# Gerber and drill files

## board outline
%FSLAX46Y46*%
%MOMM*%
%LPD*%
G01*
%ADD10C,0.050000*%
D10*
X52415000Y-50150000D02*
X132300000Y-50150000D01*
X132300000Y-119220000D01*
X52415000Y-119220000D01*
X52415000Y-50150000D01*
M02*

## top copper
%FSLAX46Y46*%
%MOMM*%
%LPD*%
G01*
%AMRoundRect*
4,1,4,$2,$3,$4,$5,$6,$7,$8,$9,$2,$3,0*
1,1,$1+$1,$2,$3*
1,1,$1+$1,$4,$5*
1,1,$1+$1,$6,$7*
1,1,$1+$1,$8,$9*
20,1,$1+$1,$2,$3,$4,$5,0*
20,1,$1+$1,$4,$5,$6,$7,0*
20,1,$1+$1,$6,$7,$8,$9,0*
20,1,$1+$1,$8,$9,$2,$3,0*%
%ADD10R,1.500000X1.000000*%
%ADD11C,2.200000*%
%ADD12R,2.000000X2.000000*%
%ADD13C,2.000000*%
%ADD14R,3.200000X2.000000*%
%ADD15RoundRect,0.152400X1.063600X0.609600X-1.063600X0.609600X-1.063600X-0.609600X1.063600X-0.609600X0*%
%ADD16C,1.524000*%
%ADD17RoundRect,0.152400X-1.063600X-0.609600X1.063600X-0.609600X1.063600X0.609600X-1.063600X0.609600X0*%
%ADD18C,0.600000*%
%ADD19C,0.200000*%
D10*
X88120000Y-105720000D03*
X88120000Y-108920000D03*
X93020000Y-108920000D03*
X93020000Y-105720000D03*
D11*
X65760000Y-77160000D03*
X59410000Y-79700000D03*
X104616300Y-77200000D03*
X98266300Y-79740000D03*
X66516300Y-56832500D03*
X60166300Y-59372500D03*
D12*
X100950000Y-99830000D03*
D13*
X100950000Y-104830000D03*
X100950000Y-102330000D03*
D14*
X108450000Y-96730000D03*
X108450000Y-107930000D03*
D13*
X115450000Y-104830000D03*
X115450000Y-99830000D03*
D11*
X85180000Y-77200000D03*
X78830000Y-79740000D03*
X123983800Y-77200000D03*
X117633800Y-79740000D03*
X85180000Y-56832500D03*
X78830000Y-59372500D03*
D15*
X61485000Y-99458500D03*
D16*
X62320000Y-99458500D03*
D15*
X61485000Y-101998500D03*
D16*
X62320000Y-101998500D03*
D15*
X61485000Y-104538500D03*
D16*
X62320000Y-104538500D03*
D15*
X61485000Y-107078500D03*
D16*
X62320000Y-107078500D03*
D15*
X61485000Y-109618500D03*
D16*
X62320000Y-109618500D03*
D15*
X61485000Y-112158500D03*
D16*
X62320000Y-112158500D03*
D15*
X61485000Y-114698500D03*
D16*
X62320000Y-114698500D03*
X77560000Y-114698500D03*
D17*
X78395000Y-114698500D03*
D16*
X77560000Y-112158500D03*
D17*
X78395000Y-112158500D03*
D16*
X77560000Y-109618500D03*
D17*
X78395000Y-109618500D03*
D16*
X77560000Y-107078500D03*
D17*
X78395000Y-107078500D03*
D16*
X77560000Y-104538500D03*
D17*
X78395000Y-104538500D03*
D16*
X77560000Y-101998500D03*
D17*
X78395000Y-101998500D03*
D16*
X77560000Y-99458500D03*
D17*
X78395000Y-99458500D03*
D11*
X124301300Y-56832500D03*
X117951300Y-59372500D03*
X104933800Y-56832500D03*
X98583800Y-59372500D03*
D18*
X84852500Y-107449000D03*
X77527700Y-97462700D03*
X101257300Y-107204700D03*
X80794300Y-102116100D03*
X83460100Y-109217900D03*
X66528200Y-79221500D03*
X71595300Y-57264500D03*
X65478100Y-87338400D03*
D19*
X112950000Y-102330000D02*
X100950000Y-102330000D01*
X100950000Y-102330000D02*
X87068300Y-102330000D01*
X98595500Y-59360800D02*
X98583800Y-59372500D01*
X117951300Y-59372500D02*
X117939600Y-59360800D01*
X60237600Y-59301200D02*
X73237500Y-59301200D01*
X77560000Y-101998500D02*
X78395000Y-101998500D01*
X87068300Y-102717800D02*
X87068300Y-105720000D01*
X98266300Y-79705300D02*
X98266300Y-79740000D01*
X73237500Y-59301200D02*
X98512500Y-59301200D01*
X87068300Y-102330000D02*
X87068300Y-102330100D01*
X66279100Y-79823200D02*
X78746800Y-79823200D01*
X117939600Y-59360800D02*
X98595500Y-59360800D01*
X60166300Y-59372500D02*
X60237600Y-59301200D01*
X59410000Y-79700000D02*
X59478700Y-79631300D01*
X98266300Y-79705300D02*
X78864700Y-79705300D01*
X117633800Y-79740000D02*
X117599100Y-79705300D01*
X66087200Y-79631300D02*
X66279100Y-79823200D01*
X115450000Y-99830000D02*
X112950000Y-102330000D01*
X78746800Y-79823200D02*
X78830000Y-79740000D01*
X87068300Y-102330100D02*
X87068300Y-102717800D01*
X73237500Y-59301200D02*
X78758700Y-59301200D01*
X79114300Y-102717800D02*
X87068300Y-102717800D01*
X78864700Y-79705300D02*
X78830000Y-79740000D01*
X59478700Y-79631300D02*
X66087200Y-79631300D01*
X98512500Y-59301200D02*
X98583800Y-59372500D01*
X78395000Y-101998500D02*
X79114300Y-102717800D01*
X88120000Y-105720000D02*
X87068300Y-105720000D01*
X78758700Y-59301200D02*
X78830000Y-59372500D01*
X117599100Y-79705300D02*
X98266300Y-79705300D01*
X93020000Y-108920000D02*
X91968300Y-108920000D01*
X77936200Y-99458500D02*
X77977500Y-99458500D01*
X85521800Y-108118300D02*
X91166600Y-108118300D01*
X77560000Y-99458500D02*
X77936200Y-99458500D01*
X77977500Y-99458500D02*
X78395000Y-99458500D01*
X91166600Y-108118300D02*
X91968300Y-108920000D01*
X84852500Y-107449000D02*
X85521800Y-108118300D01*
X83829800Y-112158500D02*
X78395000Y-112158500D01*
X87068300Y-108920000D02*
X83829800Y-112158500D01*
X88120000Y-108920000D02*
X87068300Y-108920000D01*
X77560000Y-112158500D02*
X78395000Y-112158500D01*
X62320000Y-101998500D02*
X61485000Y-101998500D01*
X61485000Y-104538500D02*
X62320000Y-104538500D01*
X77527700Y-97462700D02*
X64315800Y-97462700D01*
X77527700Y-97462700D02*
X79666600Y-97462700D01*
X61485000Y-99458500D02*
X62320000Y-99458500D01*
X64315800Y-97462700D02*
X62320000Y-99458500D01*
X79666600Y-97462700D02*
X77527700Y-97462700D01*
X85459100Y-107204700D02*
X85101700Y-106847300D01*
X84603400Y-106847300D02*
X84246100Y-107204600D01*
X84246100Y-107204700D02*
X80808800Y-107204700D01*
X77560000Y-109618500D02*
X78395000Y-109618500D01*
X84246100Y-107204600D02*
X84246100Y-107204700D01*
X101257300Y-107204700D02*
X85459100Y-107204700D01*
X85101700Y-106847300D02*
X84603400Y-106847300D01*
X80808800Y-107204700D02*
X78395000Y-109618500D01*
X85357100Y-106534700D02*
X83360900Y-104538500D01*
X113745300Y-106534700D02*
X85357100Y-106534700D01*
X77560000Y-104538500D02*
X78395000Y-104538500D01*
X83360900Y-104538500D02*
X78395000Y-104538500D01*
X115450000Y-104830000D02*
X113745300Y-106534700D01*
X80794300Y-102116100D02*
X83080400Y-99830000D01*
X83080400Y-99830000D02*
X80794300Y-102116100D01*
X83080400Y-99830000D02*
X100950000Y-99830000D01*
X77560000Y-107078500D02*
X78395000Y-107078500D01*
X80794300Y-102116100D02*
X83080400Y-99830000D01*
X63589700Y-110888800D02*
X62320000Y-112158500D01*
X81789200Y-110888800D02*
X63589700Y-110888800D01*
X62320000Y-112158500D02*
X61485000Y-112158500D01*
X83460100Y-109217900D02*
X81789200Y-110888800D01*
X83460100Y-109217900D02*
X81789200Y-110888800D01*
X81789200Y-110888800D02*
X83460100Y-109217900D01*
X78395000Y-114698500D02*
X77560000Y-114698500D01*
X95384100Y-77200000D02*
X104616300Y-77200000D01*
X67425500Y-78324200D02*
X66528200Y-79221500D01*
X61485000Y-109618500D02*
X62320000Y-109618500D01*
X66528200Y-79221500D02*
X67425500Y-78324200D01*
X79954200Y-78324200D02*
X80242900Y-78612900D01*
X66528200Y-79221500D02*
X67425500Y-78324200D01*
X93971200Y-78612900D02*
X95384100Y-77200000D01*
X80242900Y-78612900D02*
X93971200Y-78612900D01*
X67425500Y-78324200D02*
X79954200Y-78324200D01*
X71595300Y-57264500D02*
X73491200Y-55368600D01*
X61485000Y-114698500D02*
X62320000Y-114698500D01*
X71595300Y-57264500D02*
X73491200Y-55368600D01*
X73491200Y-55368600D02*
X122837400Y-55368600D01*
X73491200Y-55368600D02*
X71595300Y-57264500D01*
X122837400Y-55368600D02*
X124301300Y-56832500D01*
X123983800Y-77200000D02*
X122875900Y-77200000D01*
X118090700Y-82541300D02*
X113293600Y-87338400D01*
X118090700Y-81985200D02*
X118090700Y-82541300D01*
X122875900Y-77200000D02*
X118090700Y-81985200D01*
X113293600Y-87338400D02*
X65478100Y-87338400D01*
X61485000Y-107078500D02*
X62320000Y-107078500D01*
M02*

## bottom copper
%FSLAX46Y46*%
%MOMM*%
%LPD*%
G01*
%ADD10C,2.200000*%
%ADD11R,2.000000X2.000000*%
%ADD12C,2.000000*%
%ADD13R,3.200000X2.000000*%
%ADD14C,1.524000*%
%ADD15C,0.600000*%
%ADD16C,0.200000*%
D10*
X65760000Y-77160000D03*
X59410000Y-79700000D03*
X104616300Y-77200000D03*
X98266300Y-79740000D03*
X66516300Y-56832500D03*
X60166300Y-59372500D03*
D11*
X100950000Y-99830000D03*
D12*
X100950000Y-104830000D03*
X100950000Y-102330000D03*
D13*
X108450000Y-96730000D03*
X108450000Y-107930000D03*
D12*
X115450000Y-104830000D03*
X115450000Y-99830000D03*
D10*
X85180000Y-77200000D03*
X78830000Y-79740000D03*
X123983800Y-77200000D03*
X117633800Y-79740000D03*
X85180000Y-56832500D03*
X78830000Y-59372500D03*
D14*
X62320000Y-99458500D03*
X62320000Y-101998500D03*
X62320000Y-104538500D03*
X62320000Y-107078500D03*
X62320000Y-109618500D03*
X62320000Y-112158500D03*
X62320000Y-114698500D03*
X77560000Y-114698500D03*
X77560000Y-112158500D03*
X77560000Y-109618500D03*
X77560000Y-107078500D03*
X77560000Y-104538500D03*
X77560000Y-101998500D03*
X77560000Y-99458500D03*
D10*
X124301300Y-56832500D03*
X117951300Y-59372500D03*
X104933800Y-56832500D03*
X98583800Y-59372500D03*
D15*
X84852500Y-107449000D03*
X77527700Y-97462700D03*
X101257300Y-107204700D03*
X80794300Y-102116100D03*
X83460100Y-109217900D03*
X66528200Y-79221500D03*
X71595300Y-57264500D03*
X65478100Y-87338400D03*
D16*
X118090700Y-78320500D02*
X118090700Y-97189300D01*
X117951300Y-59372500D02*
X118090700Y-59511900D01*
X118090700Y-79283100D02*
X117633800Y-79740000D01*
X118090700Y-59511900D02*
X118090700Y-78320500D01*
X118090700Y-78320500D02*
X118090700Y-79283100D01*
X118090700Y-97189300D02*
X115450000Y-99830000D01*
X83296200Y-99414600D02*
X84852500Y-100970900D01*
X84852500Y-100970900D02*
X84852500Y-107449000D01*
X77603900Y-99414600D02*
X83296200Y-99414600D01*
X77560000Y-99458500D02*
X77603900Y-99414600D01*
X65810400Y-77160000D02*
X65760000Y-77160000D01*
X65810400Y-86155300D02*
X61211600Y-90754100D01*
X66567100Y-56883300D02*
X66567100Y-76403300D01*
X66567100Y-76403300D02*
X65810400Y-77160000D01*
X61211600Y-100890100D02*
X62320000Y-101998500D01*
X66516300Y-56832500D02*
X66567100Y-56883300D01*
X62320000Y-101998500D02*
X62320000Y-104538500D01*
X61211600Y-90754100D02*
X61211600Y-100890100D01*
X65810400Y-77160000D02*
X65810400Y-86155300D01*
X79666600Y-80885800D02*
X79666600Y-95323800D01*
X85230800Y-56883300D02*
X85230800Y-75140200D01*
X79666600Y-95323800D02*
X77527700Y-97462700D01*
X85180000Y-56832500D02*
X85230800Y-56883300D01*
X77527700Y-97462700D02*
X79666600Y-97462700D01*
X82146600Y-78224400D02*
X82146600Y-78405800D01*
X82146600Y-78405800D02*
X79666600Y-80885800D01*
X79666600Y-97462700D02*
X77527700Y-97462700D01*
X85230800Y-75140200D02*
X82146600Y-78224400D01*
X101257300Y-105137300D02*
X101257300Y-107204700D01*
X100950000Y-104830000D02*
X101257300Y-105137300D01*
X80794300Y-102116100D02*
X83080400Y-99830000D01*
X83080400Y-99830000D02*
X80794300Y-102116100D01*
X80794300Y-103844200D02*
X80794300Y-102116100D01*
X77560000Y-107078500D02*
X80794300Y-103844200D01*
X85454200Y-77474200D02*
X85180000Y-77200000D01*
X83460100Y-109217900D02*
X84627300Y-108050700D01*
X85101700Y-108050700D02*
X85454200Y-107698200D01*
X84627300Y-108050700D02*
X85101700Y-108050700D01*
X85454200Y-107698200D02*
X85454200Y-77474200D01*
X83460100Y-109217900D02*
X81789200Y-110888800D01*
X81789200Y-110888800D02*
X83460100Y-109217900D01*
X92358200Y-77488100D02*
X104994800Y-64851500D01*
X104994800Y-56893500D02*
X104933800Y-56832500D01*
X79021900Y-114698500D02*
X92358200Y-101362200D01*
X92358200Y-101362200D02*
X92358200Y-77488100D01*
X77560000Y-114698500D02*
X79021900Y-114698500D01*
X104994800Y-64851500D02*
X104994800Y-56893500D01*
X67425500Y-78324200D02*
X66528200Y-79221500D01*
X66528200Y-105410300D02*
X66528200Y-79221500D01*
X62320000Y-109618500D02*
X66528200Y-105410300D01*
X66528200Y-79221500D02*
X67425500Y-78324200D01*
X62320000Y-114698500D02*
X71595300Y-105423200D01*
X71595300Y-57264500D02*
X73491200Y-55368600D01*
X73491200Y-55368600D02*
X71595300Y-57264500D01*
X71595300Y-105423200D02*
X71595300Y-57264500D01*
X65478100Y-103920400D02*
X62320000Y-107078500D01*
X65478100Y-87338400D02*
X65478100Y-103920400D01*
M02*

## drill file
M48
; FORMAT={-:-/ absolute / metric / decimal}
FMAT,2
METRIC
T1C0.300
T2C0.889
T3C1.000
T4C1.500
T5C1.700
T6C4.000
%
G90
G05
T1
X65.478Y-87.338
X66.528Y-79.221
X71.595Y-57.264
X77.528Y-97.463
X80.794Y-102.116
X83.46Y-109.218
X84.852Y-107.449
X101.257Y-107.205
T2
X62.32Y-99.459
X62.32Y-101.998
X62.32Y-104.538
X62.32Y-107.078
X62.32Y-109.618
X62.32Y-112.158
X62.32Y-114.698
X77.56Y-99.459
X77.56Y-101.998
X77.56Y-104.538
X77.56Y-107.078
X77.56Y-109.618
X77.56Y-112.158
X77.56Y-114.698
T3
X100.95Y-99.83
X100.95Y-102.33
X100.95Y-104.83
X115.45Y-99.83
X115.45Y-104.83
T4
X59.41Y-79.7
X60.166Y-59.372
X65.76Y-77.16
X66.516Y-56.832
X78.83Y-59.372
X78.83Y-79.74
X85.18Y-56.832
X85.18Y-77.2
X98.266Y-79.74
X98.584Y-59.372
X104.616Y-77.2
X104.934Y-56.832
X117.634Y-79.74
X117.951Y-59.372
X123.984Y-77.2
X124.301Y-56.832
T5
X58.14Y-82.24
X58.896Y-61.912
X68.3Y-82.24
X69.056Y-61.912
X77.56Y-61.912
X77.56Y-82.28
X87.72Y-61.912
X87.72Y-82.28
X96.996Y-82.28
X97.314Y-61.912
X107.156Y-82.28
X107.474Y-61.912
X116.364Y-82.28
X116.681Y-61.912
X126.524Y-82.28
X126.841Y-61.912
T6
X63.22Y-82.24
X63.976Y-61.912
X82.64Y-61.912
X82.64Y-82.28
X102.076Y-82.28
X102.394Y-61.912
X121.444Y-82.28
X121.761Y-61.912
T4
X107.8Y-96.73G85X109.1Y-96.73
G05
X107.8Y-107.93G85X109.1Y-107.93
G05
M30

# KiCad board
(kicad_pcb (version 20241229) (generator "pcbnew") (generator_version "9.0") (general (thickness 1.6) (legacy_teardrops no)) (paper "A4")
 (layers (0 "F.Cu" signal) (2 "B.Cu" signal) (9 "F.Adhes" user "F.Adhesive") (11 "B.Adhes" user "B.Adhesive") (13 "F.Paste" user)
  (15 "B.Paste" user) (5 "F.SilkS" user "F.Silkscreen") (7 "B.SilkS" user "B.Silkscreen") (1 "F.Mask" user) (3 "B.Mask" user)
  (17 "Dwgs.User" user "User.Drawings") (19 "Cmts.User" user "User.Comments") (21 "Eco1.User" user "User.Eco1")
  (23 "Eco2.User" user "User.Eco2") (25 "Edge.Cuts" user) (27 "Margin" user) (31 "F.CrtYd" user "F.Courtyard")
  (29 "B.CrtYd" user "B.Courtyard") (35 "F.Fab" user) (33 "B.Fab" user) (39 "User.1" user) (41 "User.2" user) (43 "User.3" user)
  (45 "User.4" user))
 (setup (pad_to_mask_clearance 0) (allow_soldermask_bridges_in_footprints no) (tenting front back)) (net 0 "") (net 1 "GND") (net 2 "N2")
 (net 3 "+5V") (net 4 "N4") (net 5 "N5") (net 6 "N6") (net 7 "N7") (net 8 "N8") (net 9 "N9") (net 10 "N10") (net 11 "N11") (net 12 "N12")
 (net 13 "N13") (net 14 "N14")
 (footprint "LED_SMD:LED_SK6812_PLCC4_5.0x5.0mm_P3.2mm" (layer "F.Cu") (at 90.57 107.32)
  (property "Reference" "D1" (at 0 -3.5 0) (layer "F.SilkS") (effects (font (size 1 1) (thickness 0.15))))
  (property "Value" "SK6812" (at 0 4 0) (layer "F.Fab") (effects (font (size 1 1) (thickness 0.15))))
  (pad "1" smd rect (at -2.45 -1.6 180) (size 1.5 1) (layers "F.Cu" "F.Mask" "F.Paste") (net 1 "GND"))
  (pad "2" smd rect (at -2.45 1.6 180) (size 1.5 1) (layers "F.Cu" "F.Mask" "F.Paste") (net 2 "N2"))
  (pad "3" smd rect (at 2.45 1.6 180) (size 1.5 1) (layers "F.Cu" "F.Mask" "F.Paste") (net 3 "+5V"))
  (pad "4" smd rect (at 2.45 -1.6 180) (size 1.5 1) (layers "F.Cu" "F.Mask" "F.Paste") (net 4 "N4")))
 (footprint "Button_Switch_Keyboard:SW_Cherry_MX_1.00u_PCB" (layer "F.Cu") (at 65.76 77.16)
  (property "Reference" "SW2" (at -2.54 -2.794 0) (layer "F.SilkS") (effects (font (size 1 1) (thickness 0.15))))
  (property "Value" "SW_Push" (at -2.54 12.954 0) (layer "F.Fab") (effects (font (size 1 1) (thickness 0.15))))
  (pad "" np_thru_hole circle (at -7.62 5.08) (size 1.7 1.7) (drill 1.7) (layers "*.Cu" "*.Mask"))
  (pad "" np_thru_hole circle (at -2.54 5.08) (size 4 4) (drill 4) (layers "*.Cu" "*.Mask"))
  (pad "" np_thru_hole circle (at 2.54 5.08) (size 1.7 1.7) (drill 1.7) (layers "*.Cu" "*.Mask"))
  (pad "1" thru_hole circle (at 0 0) (size 2.2 2.2) (drill 1.5) (layers "*.Cu" "*.Mask") (remove_unused_layers no) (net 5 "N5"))
  (pad "2" thru_hole circle (at -6.35 2.54) (size 2.2 2.2) (drill 1.5) (layers "*.Cu" "*.Mask") (remove_unused_layers no) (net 1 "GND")))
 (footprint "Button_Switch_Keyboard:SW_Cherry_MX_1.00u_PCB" (layer "F.Cu") (at 104.6163 77.2)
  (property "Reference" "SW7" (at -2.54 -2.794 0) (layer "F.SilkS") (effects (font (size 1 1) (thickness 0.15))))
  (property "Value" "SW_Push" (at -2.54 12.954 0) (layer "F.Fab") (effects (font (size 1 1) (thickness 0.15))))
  (pad "" np_thru_hole circle (at -7.62 5.08) (size 1.7 1.7) (drill 1.7) (layers "*.Cu" "*.Mask"))
  (pad "" np_thru_hole circle (at -2.54 5.08) (size 4 4) (drill 4) (layers "*.Cu" "*.Mask"))
  (pad "" np_thru_hole circle (at 2.54 5.08) (size 1.7 1.7) (drill 1.7) (layers "*.Cu" "*.Mask"))
  (pad "1" thru_hole circle (at 0 0) (size 2.2 2.2) (drill 1.5) (layers "*.Cu" "*.Mask") (remove_unused_layers no) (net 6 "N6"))
  (pad "2" thru_hole circle (at -6.35 2.54) (size 2.2 2.2) (drill 1.5) (layers "*.Cu" "*.Mask") (remove_unused_layers no) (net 1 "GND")))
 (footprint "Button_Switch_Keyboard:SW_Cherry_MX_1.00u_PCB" (layer "F.Cu") (at 66.5163 56.8325)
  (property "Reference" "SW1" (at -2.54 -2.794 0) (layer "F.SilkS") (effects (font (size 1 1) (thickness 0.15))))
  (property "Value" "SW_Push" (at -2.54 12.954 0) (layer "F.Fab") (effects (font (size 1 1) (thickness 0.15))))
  (pad "" np_thru_hole circle (at -7.62 5.08) (size 1.7 1.7) (drill 1.7) (layers "*.Cu" "*.Mask"))
  (pad "" np_thru_hole circle (at -2.54 5.08) (size 4 4) (drill 4) (layers "*.Cu" "*.Mask"))
  (pad "" np_thru_hole circle (at 2.54 5.08) (size 1.7 1.7) (drill 1.7) (layers "*.Cu" "*.Mask"))
  (pad "1" thru_hole circle (at 0 0) (size 2.2 2.2) (drill 1.5) (layers "*.Cu" "*.Mask") (remove_unused_layers no) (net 5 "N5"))
  (pad "2" thru_hole circle (at -6.35 2.54) (size 2.2 2.2) (drill 1.5) (layers "*.Cu" "*.Mask") (remove_unused_layers no) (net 1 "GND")))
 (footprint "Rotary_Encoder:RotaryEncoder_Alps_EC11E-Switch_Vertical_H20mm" (layer "F.Cu") (at 100.95 99.83)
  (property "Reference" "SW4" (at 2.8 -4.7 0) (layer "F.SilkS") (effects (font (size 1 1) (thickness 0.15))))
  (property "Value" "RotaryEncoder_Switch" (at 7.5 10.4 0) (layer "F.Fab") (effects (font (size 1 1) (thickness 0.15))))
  (pad "A" thru_hole rect (at 0 0) (size 2 2) (drill 1) (layers "*.Cu" "*.Mask") (remove_unused_layers no) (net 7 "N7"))
  (pad "B" thru_hole circle (at 0 5) (size 2 2) (drill 1) (layers "*.Cu" "*.Mask") (remove_unused_layers no) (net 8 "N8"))
  (pad "C" thru_hole circle (at 0 2.5) (size 2 2) (drill 1) (layers "*.Cu" "*.Mask") (remove_unused_layers no) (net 1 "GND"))
  (pad "MP" thru_hole rect (at 7.5 -3.1) (size 3.2 2) (drill oval 2.8 1.5) (layers "*.Cu" "*.Mask") (remove_unused_layers no))
  (pad "MP" thru_hole rect (at 7.5 8.1) (size 3.2 2) (drill oval 2.8 1.5) (layers "*.Cu" "*.Mask") (remove_unused_layers no))
  (pad "S1" thru_hole circle (at 14.5 5) (size 2 2) (drill 1) (layers "*.Cu" "*.Mask") (remove_unused_layers no) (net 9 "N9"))
  (pad "S2" thru_hole circle (at 14.5 0) (size 2 2) (drill 1) (layers "*.Cu" "*.Mask") (remove_unused_layers no) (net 1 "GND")))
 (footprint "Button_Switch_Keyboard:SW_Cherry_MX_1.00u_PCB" (layer "F.Cu") (at 85.18 77.2)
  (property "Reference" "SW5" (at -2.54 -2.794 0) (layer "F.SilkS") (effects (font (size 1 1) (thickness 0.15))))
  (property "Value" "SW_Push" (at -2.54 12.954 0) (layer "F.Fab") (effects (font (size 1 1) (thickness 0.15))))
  (pad "" np_thru_hole circle (at -7.62 5.08) (size 1.7 1.7) (drill 1.7) (layers "*.Cu" "*.Mask"))
  (pad "" np_thru_hole circle (at -2.54 5.08) (size 4 4) (drill 4) (layers "*.Cu" "*.Mask"))
  (pad "" np_thru_hole circle (at 2.54 5.08) (size 1.7 1.7) (drill 1.7) (layers "*.Cu" "*.Mask"))
  (pad "1" thru_hole circle (at 0 0) (size 2.2 2.2) (drill 1.5) (layers "*.Cu" "*.Mask") (remove_unused_layers no) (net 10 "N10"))
  (pad "2" thru_hole circle (at -6.35 2.54) (size 2.2 2.2) (drill 1.5) (layers "*.Cu" "*.Mask") (remove_unused_layers no) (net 1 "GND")))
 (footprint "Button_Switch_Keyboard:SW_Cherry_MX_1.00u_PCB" (layer "F.Cu") (at 123.9838 77.2)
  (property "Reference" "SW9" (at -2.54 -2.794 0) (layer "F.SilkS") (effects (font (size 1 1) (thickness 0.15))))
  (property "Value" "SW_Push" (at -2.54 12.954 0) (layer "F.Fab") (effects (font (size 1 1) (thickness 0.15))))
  (pad "" np_thru_hole circle (at -7.62 5.08) (size 1.7 1.7) (drill 1.7) (layers "*.Cu" "*.Mask"))
  (pad "" np_thru_hole circle (at -2.54 5.08) (size 4 4) (drill 4) (layers "*.Cu" "*.Mask"))
  (pad "" np_thru_hole circle (at 2.54 5.08) (size 1.7 1.7) (drill 1.7) (layers "*.Cu" "*.Mask"))
  (pad "1" thru_hole circle (at 0 0) (size 2.2 2.2) (drill 1.5) (layers "*.Cu" "*.Mask") (remove_unused_layers no) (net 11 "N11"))
  (pad "2" thru_hole circle (at -6.35 2.54) (size 2.2 2.2) (drill 1.5) (layers "*.Cu" "*.Mask") (remove_unused_layers no) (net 1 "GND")))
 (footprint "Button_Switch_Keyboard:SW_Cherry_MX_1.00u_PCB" (layer "F.Cu") (at 85.18 56.8325)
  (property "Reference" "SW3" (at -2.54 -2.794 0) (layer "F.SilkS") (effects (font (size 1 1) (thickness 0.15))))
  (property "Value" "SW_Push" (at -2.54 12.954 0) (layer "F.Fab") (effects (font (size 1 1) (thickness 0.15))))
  (pad "" np_thru_hole circle (at -7.62 5.08) (size 1.7 1.7) (drill 1.7) (layers "*.Cu" "*.Mask"))
  (pad "" np_thru_hole circle (at -2.54 5.08) (size 4 4) (drill 4) (layers "*.Cu" "*.Mask"))
  (pad "" np_thru_hole circle (at 2.54 5.08) (size 1.7 1.7) (drill 1.7) (layers "*.Cu" "*.Mask"))
  (pad "1" thru_hole circle (at 0 0) (size 2.2 2.2) (drill 1.5) (layers "*.Cu" "*.Mask") (remove_unused_layers no) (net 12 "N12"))
  (pad "2" thru_hole circle (at -6.35 2.54) (size 2.2 2.2) (drill 1.5) (layers "*.Cu" "*.Mask") (remove_unused_layers no) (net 1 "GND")))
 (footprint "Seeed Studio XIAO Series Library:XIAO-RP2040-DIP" (layer "F.Cu") (at 69.94 107.0785)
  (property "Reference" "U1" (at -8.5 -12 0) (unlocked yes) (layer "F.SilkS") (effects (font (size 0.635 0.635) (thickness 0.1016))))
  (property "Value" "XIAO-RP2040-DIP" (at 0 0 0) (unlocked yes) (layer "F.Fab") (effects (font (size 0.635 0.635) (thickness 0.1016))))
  (pad "1" smd roundrect (at -8.455 -7.62 180) (size 2.432 1.524) (layers "F.Cu" "F.Mask") (roundrect_rratio 0.1) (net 12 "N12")
   (thermal_bridge_angle 45))
  (pad "1" thru_hole circle (at -7.62 -7.62 180) (size 1.524 1.524) (drill 0.889) (layers "*.Cu" "*.Mask") (remove_unused_layers no)
   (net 12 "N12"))
  (pad "2" smd roundrect (at -8.455 -5.08 180) (size 2.432 1.524) (layers "F.Cu" "F.Mask") (roundrect_rratio 0.1) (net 5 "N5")
   (thermal_bridge_angle 45))
  (pad "2" thru_hole circle (at -7.62 -5.08 180) (size 1.524 1.524) (drill 0.889) (layers "*.Cu" "*.Mask") (remove_unused_layers no)
   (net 5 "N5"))
  (pad "3" smd roundrect (at -8.455 -2.54 180) (size 2.432 1.524) (layers "F.Cu" "F.Mask") (roundrect_rratio 0.1) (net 5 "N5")
   (thermal_bridge_angle 45))
  (pad "3" thru_hole circle (at -7.62 -2.54 180) (size 1.524 1.524) (drill 0.889) (layers "*.Cu" "*.Mask") (remove_unused_layers no)
   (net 5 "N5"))
  (pad "4" smd roundrect (at -8.455 0 180) (size 2.432 1.524) (layers "F.Cu" "F.Mask") (roundrect_rratio 0.1) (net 11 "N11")
   (thermal_bridge_angle 45))
  (pad "4" thru_hole circle (at -7.62 0 180) (size 1.524 1.524) (drill 0.889) (layers "*.Cu" "*.Mask") (remove_unused_layers no)
   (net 11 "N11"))
  (pad "5" smd roundrect (at -8.455 2.54 180) (size 2.432 1.524) (layers "F.Cu" "F.Mask") (roundrect_rratio 0.1) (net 6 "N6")
   (thermal_bridge_angle 45))
  (pad "5" thru_hole circle (at -7.62 2.54 180) (size 1.524 1.524) (drill 0.889) (layers "*.Cu" "*.Mask") (remove_unused_layers no)
   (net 6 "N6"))
  (pad "6" smd roundrect (at -8.455 5.08 180) (size 2.432 1.524) (layers "F.Cu" "F.Mask") (roundrect_rratio 0.1) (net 10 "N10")
   (thermal_bridge_angle 45))
  (pad "6" thru_hole circle (at -7.62 5.08 180) (size 1.524 1.524) (drill 0.889) (layers "*.Cu" "*.Mask") (remove_unused_layers no)
   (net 10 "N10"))
  (pad "7" smd roundrect (at -8.455 7.62 180) (size 2.432 1.524) (layers "F.Cu" "F.Mask") (roundrect_rratio 0.1) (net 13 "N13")
   (thermal_bridge_angle 45))
  (pad "7" thru_hole circle (at -7.62 7.62 180) (size 1.524 1.524) (drill 0.889) (layers "*.Cu" "*.Mask") (remove_unused_layers no)
   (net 13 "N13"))
  (pad "8" thru_hole circle (at 7.62 7.62) (size 1.524 1.524) (drill 0.889) (layers "*.Cu" "*.Mask") (remove_unused_layers no)
   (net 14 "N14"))
  (pad "8" smd roundrect (at 8.455 7.62) (size 2.432 1.524) (layers "F.Cu" "F.Mask") (roundrect_rratio 0.1) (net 14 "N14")
   (thermal_bridge_angle 45))
  (pad "9" thru_hole circle (at 7.62 5.08) (size 1.524 1.524) (drill 0.889) (layers "*.Cu" "*.Mask") (remove_unused_layers no) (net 2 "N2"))
  (pad "9" smd roundrect (at 8.455 5.08) (size 2.432 1.524) (layers "F.Cu" "F.Mask") (roundrect_rratio 0.1) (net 2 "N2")
   (thermal_bridge_angle 45))
  (pad "10" thru_hole circle (at 7.62 2.54) (size 1.524 1.524) (drill 0.889) (layers "*.Cu" "*.Mask") (remove_unused_layers no) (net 8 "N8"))
  (pad "10" smd roundrect (at 8.455 2.54) (size 2.432 1.524) (layers "F.Cu" "F.Mask") (roundrect_rratio 0.1) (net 8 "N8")
   (thermal_bridge_angle 45))
  (pad "11" thru_hole circle (at 7.62 0) (size 1.524 1.524) (drill 0.889) (layers "*.Cu" "*.Mask") (remove_unused_layers no) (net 7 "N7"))
  (pad "11" smd roundrect (at 8.455 0) (size 2.432 1.524) (layers "F.Cu" "F.Mask") (roundrect_rratio 0.1) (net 7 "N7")
   (thermal_bridge_angle 45))
  (pad "12" thru_hole circle (at 7.62 -2.54) (size 1.524 1.524) (drill 0.889) (layers "*.Cu" "*.Mask") (remove_unused_layers no)
   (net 9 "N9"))
  (pad "12" smd roundrect (at 8.455 -2.54) (size 2.432 1.524) (layers "F.Cu" "F.Mask") (roundrect_rratio 0.1) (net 9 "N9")
   (thermal_bridge_angle 45))
  (pad "13" thru_hole circle (at 7.62 -5.08) (size 1.524 1.524) (drill 0.889) (layers "*.Cu" "*.Mask") (remove_unused_layers no)
   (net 1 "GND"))
  (pad "13" smd roundrect (at 8.455 -5.08) (size 2.432 1.524) (layers "F.Cu" "F.Mask") (roundrect_rratio 0.1) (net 1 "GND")
   (thermal_bridge_angle 45))
  (pad "14" thru_hole circle (at 7.62 -7.62) (size 1.524 1.524) (drill 0.889) (layers "*.Cu" "*.Mask") (remove_unused_layers no)
   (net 3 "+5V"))
  (pad "14" smd roundrect (at 8.455 -7.62) (size 2.432 1.524) (layers "F.Cu" "F.Mask") (roundrect_rratio 0.1) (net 3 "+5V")
   (thermal_bridge_angle 45)))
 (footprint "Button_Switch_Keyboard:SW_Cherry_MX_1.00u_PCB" (layer "F.Cu") (at 124.3013 56.8325)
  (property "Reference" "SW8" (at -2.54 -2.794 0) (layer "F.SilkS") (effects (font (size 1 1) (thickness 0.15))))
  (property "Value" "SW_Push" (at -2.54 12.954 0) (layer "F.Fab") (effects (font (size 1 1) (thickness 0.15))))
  (pad "" np_thru_hole circle (at -7.62 5.08) (size 1.7 1.7) (drill 1.7) (layers "*.Cu" "*.Mask"))
  (pad "" np_thru_hole circle (at -2.54 5.08) (size 4 4) (drill 4) (layers "*.Cu" "*.Mask"))
  (pad "" np_thru_hole circle (at 2.54 5.08) (size 1.7 1.7) (drill 1.7) (layers "*.Cu" "*.Mask"))
  (pad "1" thru_hole circle (at 0 0) (size 2.2 2.2) (drill 1.5) (layers "*.Cu" "*.Mask") (remove_unused_layers no) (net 13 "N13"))
  (pad "2" thru_hole circle (at -6.35 2.54) (size 2.2 2.2) (drill 1.5) (layers "*.Cu" "*.Mask") (remove_unused_layers no) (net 1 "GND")))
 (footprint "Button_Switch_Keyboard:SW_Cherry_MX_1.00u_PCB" (layer "F.Cu") (at 104.9338 56.8325)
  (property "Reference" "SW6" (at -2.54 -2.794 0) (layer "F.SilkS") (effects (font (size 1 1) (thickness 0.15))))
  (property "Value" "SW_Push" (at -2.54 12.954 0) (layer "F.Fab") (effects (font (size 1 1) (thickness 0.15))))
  (pad "" np_thru_hole circle (at -7.62 5.08) (size 1.7 1.7) (drill 1.7) (layers "*.Cu" "*.Mask"))
  (pad "" np_thru_hole circle (at -2.54 5.08) (size 4 4) (drill 4) (layers "*.Cu" "*.Mask"))
  (pad "" np_thru_hole circle (at 2.54 5.08) (size 1.7 1.7) (drill 1.7) (layers "*.Cu" "*.Mask"))
  (pad "1" thru_hole circle (at 0 0) (size 2.2 2.2) (drill 1.5) (layers "*.Cu" "*.Mask") (remove_unused_layers no) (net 14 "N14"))
  (pad "2" thru_hole circle (at -6.35 2.54) (size 2.2 2.2) (drill 1.5) (layers "*.Cu" "*.Mask") (remove_unused_layers no) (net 1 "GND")))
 (gr_rect (start 52.415 50.15) (end 132.3 119.22) (stroke (width 0.05) (type default)) (fill no) (layer "Edge.Cuts"))
 (segment (start 112.95 102.33) (end 100.95 102.33) (width 0.2) (layer "F.Cu") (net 1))
 (segment (start 100.95 102.33) (end 87.0683 102.33) (width 0.2) (layer "F.Cu") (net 1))
 (segment (start 98.5955 59.3608) (end 98.5838 59.3725) (width 0.2) (layer "F.Cu") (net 1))
 (segment (start 117.9513 59.3725) (end 117.9396 59.3608) (width 0.2) (layer "F.Cu") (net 1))
 (segment (start 60.2376 59.3012) (end 73.2375 59.3012) (width 0.2) (layer "F.Cu") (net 1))
 (segment (start 77.56 101.9985) (end 78.395 101.9985) (width 0.2) (layer "F.Cu") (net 1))
 (segment (start 87.0683 102.7178) (end 87.0683 105.72) (width 0.2) (layer "F.Cu") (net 1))
 (segment (start 98.2663 79.7053) (end 98.2663 79.74) (width 0.2) (layer "F.Cu") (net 1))
 (segment (start 73.2375 59.3012) (end 98.5125 59.3012) (width 0.2) (layer "F.Cu") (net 1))
 (segment (start 87.0683 102.33) (end 87.0683 102.3301) (width 0.2) (layer "F.Cu") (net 1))
 (segment (start 66.2791 79.8232) (end 78.7468 79.8232) (width 0.2) (layer "F.Cu") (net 1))
 (segment (start 117.9396 59.3608) (end 98.5955 59.3608) (width 0.2) (layer "F.Cu") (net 1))
 (segment (start 60.1663 59.3725) (end 60.2376 59.3012) (width 0.2) (layer "F.Cu") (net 1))
 (segment (start 59.41 79.7) (end 59.4787 79.6313) (width 0.2) (layer "F.Cu") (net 1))
 (segment (start 98.2663 79.7053) (end 78.8647 79.7053) (width 0.2) (layer "F.Cu") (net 1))
 (segment (start 117.6338 79.74) (end 117.5991 79.7053) (width 0.2) (layer "F.Cu") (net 1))
 (segment (start 66.0872 79.6313) (end 66.2791 79.8232) (width 0.2) (layer "F.Cu") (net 1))
 (segment (start 115.45 99.83) (end 112.95 102.33) (width 0.2) (layer "F.Cu") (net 1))
 (segment (start 78.7468 79.8232) (end 78.83 79.74) (width 0.2) (layer "F.Cu") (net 1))
 (segment (start 87.0683 102.3301) (end 87.0683 102.7178) (width 0.2) (layer "F.Cu") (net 1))
 (segment (start 73.2375 59.3012) (end 78.7587 59.3012) (width 0.2) (layer "F.Cu") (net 1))
 (segment (start 79.1143 102.7178) (end 87.0683 102.7178) (width 0.2) (layer "F.Cu") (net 1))
 (segment (start 78.8647 79.7053) (end 78.83 79.74) (width 0.2) (layer "F.Cu") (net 1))
 (segment (start 59.4787 79.6313) (end 66.0872 79.6313) (width 0.2) (layer "F.Cu") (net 1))
 (segment (start 98.5125 59.3012) (end 98.5838 59.3725) (width 0.2) (layer "F.Cu") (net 1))
 (segment (start 78.395 101.9985) (end 79.1143 102.7178) (width 0.2) (layer "F.Cu") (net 1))
 (segment (start 88.12 105.72) (end 87.0683 105.72) (width 0.2) (layer "F.Cu") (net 1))
 (segment (start 78.7587 59.3012) (end 78.83 59.3725) (width 0.2) (layer "F.Cu") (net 1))
 (segment (start 117.5991 79.7053) (end 98.2663 79.7053) (width 0.2) (layer "F.Cu") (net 1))
 (segment (start 118.0907 78.3205) (end 118.0907 97.1893) (width 0.2) (layer "B.Cu") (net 1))
 (segment (start 117.9513 59.3725) (end 118.0907 59.5119) (width 0.2) (layer "B.Cu") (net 1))
 (segment (start 118.0907 79.2831) (end 117.6338 79.74) (width 0.2) (layer "B.Cu") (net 1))
 (segment (start 118.0907 59.5119) (end 118.0907 78.3205) (width 0.2) (layer "B.Cu") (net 1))
 (segment (start 118.0907 78.3205) (end 118.0907 79.2831) (width 0.2) (layer "B.Cu") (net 1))
 (segment (start 118.0907 97.1893) (end 115.45 99.83) (width 0.2) (layer "B.Cu") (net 1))
 (segment (start 93.02 108.92) (end 91.9683 108.92) (width 0.2) (layer "F.Cu") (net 3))
 (segment (start 77.9362 99.4585) (end 77.9775 99.4585) (width 0.2) (layer "F.Cu") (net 3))
 (segment (start 85.5218 108.1183) (end 91.1666 108.1183) (width 0.2) (layer "F.Cu") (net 3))
 (segment (start 77.56 99.4585) (end 77.9362 99.4585) (width 0.2) (layer "F.Cu") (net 3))
 (segment (start 77.9775 99.4585) (end 78.395 99.4585) (width 0.2) (layer "F.Cu") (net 3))
 (segment (start 91.1666 108.1183) (end 91.9683 108.92) (width 0.2) (layer "F.Cu") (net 3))
 (segment (start 84.8525 107.449) (end 85.5218 108.1183) (width 0.2) (layer "F.Cu") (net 3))
 (via (at 84.8525 107.449) (size 0.6) (drill 0.3) (layers "F.Cu" "B.Cu") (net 3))
 (segment (start 83.2962 99.4146) (end 84.8525 100.9709) (width 0.2) (layer "B.Cu") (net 3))
 (segment (start 84.8525 100.9709) (end 84.8525 107.449) (width 0.2) (layer "B.Cu") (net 3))
 (segment (start 77.6039 99.4146) (end 83.2962 99.4146) (width 0.2) (layer "B.Cu") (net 3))
 (segment (start 77.56 99.4585) (end 77.6039 99.4146) (width 0.2) (layer "B.Cu") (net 3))
 (segment (start 83.8298 112.1585) (end 78.395 112.1585) (width 0.2) (layer "F.Cu") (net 2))
 (segment (start 87.0683 108.92) (end 83.8298 112.1585) (width 0.2) (layer "F.Cu") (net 2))
 (segment (start 88.12 108.92) (end 87.0683 108.92) (width 0.2) (layer "F.Cu") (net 2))
 (segment (start 77.56 112.1585) (end 78.395 112.1585) (width 0.2) (layer "F.Cu") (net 2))
 (segment (start 62.32 101.9985) (end 61.485 101.9985) (width 0.2) (layer "F.Cu") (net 5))
 (segment (start 61.485 104.5385) (end 62.32 104.5385) (width 0.2) (layer "F.Cu") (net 5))
 (segment (start 65.8104 77.16) (end 65.76 77.16) (width 0.2) (layer "B.Cu") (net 5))
 (segment (start 65.8104 86.1553) (end 61.2116 90.7541) (width 0.2) (layer "B.Cu") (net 5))
 (segment (start 66.5671 56.8833) (end 66.5671 76.4033) (width 0.2) (layer "B.Cu") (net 5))
 (segment (start 66.5671 76.4033) (end 65.8104 77.16) (width 0.2) (layer "B.Cu") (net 5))
 (segment (start 61.2116 100.8901) (end 62.32 101.9985) (width 0.2) (layer "B.Cu") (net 5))
 (segment (start 66.5163 56.8325) (end 66.5671 56.8833) (width 0.2) (layer "B.Cu") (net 5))
 (segment (start 62.32 101.9985) (end 62.32 104.5385) (width 0.2) (layer "B.Cu") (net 5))
 (segment (start 61.2116 90.7541) (end 61.2116 100.8901) (width 0.2) (layer "B.Cu") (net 5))
 (segment (start 65.8104 77.16) (end 65.8104 86.1553) (width 0.2) (layer "B.Cu") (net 5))
 (segment (start 77.5277 97.4627) (end 64.3158 97.4627) (width 0.2) (layer "F.Cu") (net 12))
 (segment (start 77.5277 97.4627) (end 79.6666 97.4627) (width 0.2) (layer "F.Cu") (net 12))
 (segment (start 61.485 99.4585) (end 62.32 99.4585) (width 0.2) (layer "F.Cu") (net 12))
 (segment (start 64.3158 97.4627) (end 62.32 99.4585) (width 0.2) (layer "F.Cu") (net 12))
 (segment (start 79.6666 97.4627) (end 77.5277 97.4627) (width 0.2) (layer "F.Cu") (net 12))
 (via (at 77.5277 97.4627) (size 0.6) (drill 0.3) (layers "F.Cu" "B.Cu") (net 12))
 (segment (start 79.6666 80.8858) (end 79.6666 95.3238) (width 0.2) (layer "B.Cu") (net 12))
 (segment (start 85.2308 56.8833) (end 85.2308 75.1402) (width 0.2) (layer "B.Cu") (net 12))
 (segment (start 79.6666 95.3238) (end 77.5277 97.4627) (width 0.2) (layer "B.Cu") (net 12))
 (segment (start 85.18 56.8325) (end 85.2308 56.8833) (width 0.2) (layer "B.Cu") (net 12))
 (segment (start 77.5277 97.4627) (end 79.6666 97.4627) (width 0.2) (layer "B.Cu") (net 12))
 (segment (start 82.1466 78.2244) (end 82.1466 78.4058) (width 0.2) (layer "B.Cu") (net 12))
 (segment (start 82.1466 78.4058) (end 79.6666 80.8858) (width 0.2) (layer "B.Cu") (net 12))
 (segment (start 79.6666 97.4627) (end 77.5277 97.4627) (width 0.2) (layer "B.Cu") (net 12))
 (segment (start 85.2308 75.1402) (end 82.1466 78.2244) (width 0.2) (layer "B.Cu") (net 12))
 (segment (start 85.4591 107.2047) (end 85.1017 106.8473) (width 0.2) (layer "F.Cu") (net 8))
 (segment (start 84.6034 106.8473) (end 84.2461 107.2046) (width 0.2) (layer "F.Cu") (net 8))
 (segment (start 84.2461 107.2047) (end 80.8088 107.2047) (width 0.2) (layer "F.Cu") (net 8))
 (segment (start 77.56 109.6185) (end 78.395 109.6185) (width 0.2) (layer "F.Cu") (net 8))
 (segment (start 84.2461 107.2046) (end 84.2461 107.2047) (width 0.2) (layer "F.Cu") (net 8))
 (segment (start 101.2573 107.2047) (end 85.4591 107.2047) (width 0.2) (layer "F.Cu") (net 8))
 (segment (start 85.1017 106.8473) (end 84.6034 106.8473) (width 0.2) (layer "F.Cu") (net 8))
 (segment (start 80.8088 107.2047) (end 78.395 109.6185) (width 0.2) (layer "F.Cu") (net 8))
 (via (at 101.2573 107.2047) (size 0.6) (drill 0.3) (layers "F.Cu" "B.Cu") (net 8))
 (segment (start 101.2573 105.1373) (end 101.2573 107.2047) (width 0.2) (layer "B.Cu") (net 8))
 (segment (start 100.95 104.83) (end 101.2573 105.1373) (width 0.2) (layer "B.Cu") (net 8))
 (segment (start 85.3571 106.5347) (end 83.3609 104.5385) (width 0.2) (layer "F.Cu") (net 9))
 (segment (start 113.7453 106.5347) (end 85.3571 106.5347) (width 0.2) (layer "F.Cu") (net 9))
 (segment (start 77.56 104.5385) (end 78.395 104.5385) (width 0.2) (layer "F.Cu") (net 9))
 (segment (start 83.3609 104.5385) (end 78.395 104.5385) (width 0.2) (layer "F.Cu") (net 9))
 (segment (start 115.45 104.83) (end 113.7453 106.5347) (width 0.2) (layer "F.Cu") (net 9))
 (segment (start 80.7943 102.1161) (end 83.0804 99.83) (width 0.2) (layer "F.Cu") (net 7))
 (segment (start 83.0804 99.83) (end 80.7943 102.1161) (width 0.2) (layer "F.Cu") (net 7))
 (segment (start 83.0804 99.83) (end 100.95 99.83) (width 0.2) (layer "F.Cu") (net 7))
 (segment (start 77.56 107.0785) (end 78.395 107.0785) (width 0.2) (layer "F.Cu") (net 7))
 (segment (start 80.7943 102.1161) (end 83.0804 99.83) (width 0.2) (layer "F.Cu") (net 7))
 (via (at 80.7943 102.1161) (size 0.6) (drill 0.3) (layers "F.Cu" "B.Cu") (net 7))
 (segment (start 80.7943 102.1161) (end 83.0804 99.83) (width 0.2) (layer "B.Cu") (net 7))
 (segment (start 83.0804 99.83) (end 80.7943 102.1161) (width 0.2) (layer "B.Cu") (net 7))
 (segment (start 80.7943 103.8442) (end 80.7943 102.1161) (width 0.2) (layer "B.Cu") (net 7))
 (segment (start 77.56 107.0785) (end 80.7943 103.8442) (width 0.2) (layer "B.Cu") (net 7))
 (segment (start 63.5897 110.8888) (end 62.32 112.1585) (width 0.2) (layer "F.Cu") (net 10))
 (segment (start 81.7892 110.8888) (end 63.5897 110.8888) (width 0.2) (layer "F.Cu") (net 10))
 (segment (start 62.32 112.1585) (end 61.485 112.1585) (width 0.2) (layer "F.Cu") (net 10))
 (segment (start 83.4601 109.2179) (end 81.7892 110.8888) (width 0.2) (layer "F.Cu") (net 10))
 (segment (start 83.4601 109.2179) (end 81.7892 110.8888) (width 0.2) (layer "F.Cu") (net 10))
 (segment (start 81.7892 110.8888) (end 83.4601 109.2179) (width 0.2) (layer "F.Cu") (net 10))
 (via (at 83.4601 109.2179) (size 0.6) (drill 0.3) (layers "F.Cu" "B.Cu") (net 10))
 (segment (start 85.4542 77.4742) (end 85.18 77.2) (width 0.2) (layer "B.Cu") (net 10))
 (segment (start 83.4601 109.2179) (end 84.6273 108.0507) (width 0.2) (layer "B.Cu") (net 10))
 (segment (start 85.1017 108.0507) (end 85.4542 107.6982) (width 0.2) (layer "B.Cu") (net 10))
 (segment (start 84.6273 108.0507) (end 85.1017 108.0507) (width 0.2) (layer "B.Cu") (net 10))
 (segment (start 85.4542 107.6982) (end 85.4542 77.4742) (width 0.2) (layer "B.Cu") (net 10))
 (segment (start 83.4601 109.2179) (end 81.7892 110.8888) (width 0.2) (layer "B.Cu") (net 10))
 (segment (start 81.7892 110.8888) (end 83.4601 109.2179) (width 0.2) (layer "B.Cu") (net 10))
 (segment (start 78.395 114.6985) (end 77.56 114.6985) (width 0.2) (layer "F.Cu") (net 14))
 (segment (start 92.3582 77.4881) (end 104.9948 64.8515) (width 0.2) (layer "B.Cu") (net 14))
 (segment (start 104.9948 56.8935) (end 104.9338 56.8325) (width 0.2) (layer "B.Cu") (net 14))
 (segment (start 79.0219 114.6985) (end 92.3582 101.3622) (width 0.2) (layer "B.Cu") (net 14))
 (segment (start 92.3582 101.3622) (end 92.3582 77.4881) (width 0.2) (layer "B.Cu") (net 14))
 (segment (start 77.56 114.6985) (end 79.0219 114.6985) (width 0.2) (layer "B.Cu") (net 14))
 (segment (start 104.9948 64.8515) (end 104.9948 56.8935) (width 0.2) (layer "B.Cu") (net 14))
 (segment (start 95.3841 77.2) (end 104.6163 77.2) (width 0.2) (layer "F.Cu") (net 6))
 (segment (start 67.4255 78.3242) (end 66.5282 79.2215) (width 0.2) (layer "F.Cu") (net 6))
 (segment (start 61.485 109.6185) (end 62.32 109.6185) (width 0.2) (layer "F.Cu") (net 6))
 (segment (start 66.5282 79.2215) (end 67.4255 78.3242) (width 0.2) (layer "F.Cu") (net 6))
 (segment (start 79.9542 78.3242) (end 80.2429 78.6129) (width 0.2) (layer "F.Cu") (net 6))
 (segment (start 66.5282 79.2215) (end 67.4255 78.3242) (width 0.2) (layer "F.Cu") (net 6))
 (segment (start 93.9712 78.6129) (end 95.3841 77.2) (width 0.2) (layer "F.Cu") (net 6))
 (segment (start 80.2429 78.6129) (end 93.9712 78.6129) (width 0.2) (layer "F.Cu") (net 6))
 (segment (start 67.4255 78.3242) (end 79.9542 78.3242) (width 0.2) (layer "F.Cu") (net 6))
 (via (at 66.5282 79.2215) (size 0.6) (drill 0.3) (layers "F.Cu" "B.Cu") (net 6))
 (segment (start 67.4255 78.3242) (end 66.5282 79.2215) (width 0.2) (layer "B.Cu") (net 6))
 (segment (start 66.5282 105.4103) (end 66.5282 79.2215) (width 0.2) (layer "B.Cu") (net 6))
 (segment (start 62.32 109.6185) (end 66.5282 105.4103) (width 0.2) (layer "B.Cu") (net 6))
 (segment (start 66.5282 79.2215) (end 67.4255 78.3242) (width 0.2) (layer "B.Cu") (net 6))
 (segment (start 71.5953 57.2645) (end 73.4912 55.3686) (width 0.2) (layer "F.Cu") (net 13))
 (segment (start 61.485 114.6985) (end 62.32 114.6985) (width 0.2) (layer "F.Cu") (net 13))
 (segment (start 71.5953 57.2645) (end 73.4912 55.3686) (width 0.2) (layer "F.Cu") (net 13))
 (segment (start 73.4912 55.3686) (end 122.8374 55.3686) (width 0.2) (layer "F.Cu") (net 13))
 (segment (start 73.4912 55.3686) (end 71.5953 57.2645) (width 0.2) (layer "F.Cu") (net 13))
 (segment (start 122.8374 55.3686) (end 124.3013 56.8325) (width 0.2) (layer "F.Cu") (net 13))
 (via (at 71.5953 57.2645) (size 0.6) (drill 0.3) (layers "F.Cu" "B.Cu") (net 13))
 (segment (start 62.32 114.6985) (end 71.5953 105.4232) (width 0.2) (layer "B.Cu") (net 13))
 (segment (start 71.5953 57.2645) (end 73.4912 55.3686) (width 0.2) (layer "B.Cu") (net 13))
 (segment (start 73.4912 55.3686) (end 71.5953 57.2645) (width 0.2) (layer "B.Cu") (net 13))
 (segment (start 71.5953 105.4232) (end 71.5953 57.2645) (width 0.2) (layer "B.Cu") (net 13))
 (segment (start 123.9838 77.2) (end 122.8759 77.2) (width 0.2) (layer "F.Cu") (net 11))
 (segment (start 118.0907 82.5413) (end 113.2936 87.3384) (width 0.2) (layer "F.Cu") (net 11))
 (segment (start 118.0907 81.9852) (end 118.0907 82.5413) (width 0.2) (layer "F.Cu") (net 11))
 (segment (start 122.8759 77.2) (end 118.0907 81.9852) (width 0.2) (layer "F.Cu") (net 11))
 (segment (start 113.2936 87.3384) (end 65.4781 87.3384) (width 0.2) (layer "F.Cu") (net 11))
 (segment (start 61.485 107.0785) (end 62.32 107.0785) (width 0.2) (layer "F.Cu") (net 11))
 (via (at 65.4781 87.3384) (size 0.6) (drill 0.3) (layers "F.Cu" "B.Cu") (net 11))
 (segment (start 65.4781 103.9204) (end 62.32 107.0785) (width 0.2) (layer "B.Cu") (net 11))
 (segment (start 65.4781 87.3384) (end 65.4781 103.9204) (width 0.2) (layer "B.Cu") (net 11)))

